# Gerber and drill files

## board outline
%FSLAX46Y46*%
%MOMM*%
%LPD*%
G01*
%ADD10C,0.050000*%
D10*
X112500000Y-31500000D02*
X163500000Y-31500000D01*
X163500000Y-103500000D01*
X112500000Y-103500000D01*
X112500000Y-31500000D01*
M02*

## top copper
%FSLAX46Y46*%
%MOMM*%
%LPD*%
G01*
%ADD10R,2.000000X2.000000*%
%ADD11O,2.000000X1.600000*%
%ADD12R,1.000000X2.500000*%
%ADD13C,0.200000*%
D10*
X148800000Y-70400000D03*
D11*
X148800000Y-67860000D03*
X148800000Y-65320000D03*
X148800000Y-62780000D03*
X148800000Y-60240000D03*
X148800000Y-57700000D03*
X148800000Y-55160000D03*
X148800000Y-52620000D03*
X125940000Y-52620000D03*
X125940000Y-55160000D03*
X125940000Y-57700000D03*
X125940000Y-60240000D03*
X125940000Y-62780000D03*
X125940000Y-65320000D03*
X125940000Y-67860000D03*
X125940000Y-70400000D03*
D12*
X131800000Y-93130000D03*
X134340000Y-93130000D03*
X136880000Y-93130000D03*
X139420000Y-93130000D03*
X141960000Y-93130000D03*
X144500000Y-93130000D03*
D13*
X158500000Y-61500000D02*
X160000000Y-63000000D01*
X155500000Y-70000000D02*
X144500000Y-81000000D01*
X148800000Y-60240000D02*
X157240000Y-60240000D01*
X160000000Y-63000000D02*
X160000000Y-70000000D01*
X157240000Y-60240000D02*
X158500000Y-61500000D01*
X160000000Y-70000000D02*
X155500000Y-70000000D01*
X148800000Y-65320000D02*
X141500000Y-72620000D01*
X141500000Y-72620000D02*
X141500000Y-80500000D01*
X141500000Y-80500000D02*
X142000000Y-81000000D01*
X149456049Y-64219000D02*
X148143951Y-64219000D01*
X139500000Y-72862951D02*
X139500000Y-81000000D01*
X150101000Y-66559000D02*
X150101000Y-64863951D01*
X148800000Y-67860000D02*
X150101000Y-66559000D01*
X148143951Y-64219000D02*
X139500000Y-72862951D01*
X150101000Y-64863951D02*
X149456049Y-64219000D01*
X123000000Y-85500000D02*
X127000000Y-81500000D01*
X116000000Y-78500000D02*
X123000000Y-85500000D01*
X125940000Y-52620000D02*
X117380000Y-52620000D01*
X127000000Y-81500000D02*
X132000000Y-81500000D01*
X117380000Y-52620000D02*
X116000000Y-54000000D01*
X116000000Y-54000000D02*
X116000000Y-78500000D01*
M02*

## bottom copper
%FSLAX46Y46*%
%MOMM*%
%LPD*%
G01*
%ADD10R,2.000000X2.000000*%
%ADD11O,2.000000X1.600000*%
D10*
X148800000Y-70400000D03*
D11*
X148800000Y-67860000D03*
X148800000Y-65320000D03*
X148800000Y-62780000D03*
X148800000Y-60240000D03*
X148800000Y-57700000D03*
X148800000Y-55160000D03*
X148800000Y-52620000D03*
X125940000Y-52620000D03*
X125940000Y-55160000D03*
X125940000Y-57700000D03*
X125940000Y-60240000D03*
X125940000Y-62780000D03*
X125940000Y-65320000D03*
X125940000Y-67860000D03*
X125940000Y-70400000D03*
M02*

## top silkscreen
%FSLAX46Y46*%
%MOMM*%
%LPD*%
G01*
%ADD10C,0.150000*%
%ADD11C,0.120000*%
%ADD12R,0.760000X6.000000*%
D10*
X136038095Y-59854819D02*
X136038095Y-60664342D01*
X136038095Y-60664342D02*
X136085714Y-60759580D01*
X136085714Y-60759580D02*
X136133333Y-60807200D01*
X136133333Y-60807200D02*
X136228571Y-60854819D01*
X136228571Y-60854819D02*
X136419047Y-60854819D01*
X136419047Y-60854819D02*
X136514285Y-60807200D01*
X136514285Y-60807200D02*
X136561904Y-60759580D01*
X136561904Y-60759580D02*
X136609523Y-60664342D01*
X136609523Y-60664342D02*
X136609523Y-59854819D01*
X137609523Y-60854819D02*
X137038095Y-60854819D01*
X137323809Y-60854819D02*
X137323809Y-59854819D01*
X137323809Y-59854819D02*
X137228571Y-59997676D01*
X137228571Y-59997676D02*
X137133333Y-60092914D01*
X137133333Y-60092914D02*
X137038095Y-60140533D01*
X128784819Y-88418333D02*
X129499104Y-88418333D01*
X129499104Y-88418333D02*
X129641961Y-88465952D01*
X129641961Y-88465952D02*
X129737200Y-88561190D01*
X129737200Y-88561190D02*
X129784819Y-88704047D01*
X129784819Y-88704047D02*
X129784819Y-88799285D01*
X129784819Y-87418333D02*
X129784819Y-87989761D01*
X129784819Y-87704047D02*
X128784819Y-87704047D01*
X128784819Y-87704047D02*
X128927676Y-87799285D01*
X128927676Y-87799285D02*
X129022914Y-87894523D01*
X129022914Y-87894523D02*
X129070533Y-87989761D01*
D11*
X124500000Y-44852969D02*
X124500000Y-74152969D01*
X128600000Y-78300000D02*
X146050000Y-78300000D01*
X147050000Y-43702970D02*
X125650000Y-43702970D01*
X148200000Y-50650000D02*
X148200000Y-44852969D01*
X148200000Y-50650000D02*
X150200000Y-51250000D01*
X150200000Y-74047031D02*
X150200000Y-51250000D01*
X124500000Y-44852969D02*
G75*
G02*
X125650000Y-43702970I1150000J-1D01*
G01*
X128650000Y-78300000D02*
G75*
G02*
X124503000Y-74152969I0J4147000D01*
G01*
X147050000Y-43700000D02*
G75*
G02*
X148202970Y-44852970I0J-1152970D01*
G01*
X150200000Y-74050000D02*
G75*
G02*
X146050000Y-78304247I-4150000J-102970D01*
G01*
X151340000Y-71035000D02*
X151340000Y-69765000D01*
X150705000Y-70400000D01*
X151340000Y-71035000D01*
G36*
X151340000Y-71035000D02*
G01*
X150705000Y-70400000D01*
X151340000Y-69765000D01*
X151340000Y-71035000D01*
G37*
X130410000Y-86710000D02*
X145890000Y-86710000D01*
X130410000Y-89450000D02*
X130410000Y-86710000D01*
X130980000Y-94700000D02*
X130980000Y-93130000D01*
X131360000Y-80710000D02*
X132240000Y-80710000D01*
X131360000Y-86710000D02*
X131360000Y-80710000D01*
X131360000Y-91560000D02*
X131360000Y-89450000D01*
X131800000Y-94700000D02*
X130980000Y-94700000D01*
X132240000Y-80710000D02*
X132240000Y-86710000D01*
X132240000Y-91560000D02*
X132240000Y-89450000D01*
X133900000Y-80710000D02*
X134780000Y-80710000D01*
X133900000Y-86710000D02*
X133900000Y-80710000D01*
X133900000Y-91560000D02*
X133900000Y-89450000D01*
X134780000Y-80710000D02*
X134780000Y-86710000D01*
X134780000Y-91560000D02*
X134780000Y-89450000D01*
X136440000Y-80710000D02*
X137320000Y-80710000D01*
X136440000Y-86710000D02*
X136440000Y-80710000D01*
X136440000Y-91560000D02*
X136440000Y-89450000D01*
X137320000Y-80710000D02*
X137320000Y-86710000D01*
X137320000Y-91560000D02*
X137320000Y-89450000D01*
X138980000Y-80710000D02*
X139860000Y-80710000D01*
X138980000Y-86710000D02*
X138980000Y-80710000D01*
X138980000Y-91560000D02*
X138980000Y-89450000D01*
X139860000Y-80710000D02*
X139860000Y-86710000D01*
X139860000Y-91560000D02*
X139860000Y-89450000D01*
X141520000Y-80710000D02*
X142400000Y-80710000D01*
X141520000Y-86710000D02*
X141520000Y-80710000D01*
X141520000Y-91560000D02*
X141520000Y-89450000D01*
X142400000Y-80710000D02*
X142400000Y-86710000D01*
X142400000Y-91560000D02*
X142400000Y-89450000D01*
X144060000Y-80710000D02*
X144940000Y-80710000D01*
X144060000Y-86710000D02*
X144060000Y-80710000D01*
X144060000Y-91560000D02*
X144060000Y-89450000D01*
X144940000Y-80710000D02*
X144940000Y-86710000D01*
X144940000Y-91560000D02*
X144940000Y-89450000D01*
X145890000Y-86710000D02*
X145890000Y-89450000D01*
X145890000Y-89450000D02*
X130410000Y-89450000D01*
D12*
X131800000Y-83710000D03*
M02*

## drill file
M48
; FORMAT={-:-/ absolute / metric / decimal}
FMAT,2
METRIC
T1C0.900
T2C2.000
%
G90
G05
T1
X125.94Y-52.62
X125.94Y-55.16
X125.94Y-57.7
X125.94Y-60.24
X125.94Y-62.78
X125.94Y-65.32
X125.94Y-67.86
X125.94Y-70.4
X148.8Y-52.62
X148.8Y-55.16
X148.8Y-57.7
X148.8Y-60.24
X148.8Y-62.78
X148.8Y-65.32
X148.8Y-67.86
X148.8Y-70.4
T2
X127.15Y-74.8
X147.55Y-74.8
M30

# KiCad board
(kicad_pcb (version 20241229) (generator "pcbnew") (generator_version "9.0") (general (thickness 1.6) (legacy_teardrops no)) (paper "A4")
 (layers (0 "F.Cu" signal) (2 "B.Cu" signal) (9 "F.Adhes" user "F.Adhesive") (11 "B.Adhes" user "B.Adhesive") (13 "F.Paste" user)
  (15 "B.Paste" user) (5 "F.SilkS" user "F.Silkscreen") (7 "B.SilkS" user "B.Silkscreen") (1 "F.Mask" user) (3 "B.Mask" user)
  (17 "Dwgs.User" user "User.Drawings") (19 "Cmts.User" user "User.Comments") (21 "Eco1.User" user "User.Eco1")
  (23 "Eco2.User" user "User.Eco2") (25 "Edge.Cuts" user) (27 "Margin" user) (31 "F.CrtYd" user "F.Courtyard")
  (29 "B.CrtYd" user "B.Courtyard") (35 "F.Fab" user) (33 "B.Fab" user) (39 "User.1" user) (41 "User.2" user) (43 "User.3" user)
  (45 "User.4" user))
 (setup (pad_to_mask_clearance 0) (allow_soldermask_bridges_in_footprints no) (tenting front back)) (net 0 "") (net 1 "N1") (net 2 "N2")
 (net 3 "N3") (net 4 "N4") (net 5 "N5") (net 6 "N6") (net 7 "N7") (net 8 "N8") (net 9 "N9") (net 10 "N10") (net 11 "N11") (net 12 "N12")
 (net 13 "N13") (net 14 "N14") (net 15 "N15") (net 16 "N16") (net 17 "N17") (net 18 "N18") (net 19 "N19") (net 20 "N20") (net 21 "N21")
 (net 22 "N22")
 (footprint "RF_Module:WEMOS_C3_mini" (layer "F.Cu") (at 148.8 70.4 180)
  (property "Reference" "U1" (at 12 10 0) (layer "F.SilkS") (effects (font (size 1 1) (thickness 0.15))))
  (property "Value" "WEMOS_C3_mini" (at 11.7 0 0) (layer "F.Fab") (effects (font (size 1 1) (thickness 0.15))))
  (fp_line (start 24.3 25.547031) (end 24.3 -3.752969) (stroke (width 0.12) (type solid)) (layer "F.SilkS"))
  (fp_line (start 20.2 -7.9) (end 2.75 -7.9) (stroke (width 0.12) (type solid)) (layer "F.SilkS"))
  (fp_line (start 1.75 26.69703) (end 23.15 26.69703) (stroke (width 0.12) (type solid)) (layer "F.SilkS"))
  (fp_line (start 0.6 19.75) (end 0.6 25.547031) (stroke (width 0.12) (type solid)) (layer "F.SilkS"))
  (fp_line (start 0.6 19.75) (end -1.4 19.15) (stroke (width 0.12) (type default)) (layer "F.SilkS"))
  (fp_line (start -1.4 -3.647031) (end -1.4 19.15) (stroke (width 0.12) (type solid)) (layer "F.SilkS"))
  (fp_arc (start 24.3 25.547031) (mid 23.963172 26.360203) (end 23.15 26.69703) (stroke (width 0.12) (type solid)) (layer "F.SilkS"))
  (fp_arc (start 20.15 -7.9) (mid 23.082383 -6.685361) (end 24.297 -3.752969) (stroke (width 0.12) (type solid)) (layer "F.SilkS"))
  (fp_arc (start 1.75 26.7) (mid 0.934727 26.362303) (end 0.59703 25.54703) (stroke (width 0.12) (type solid)) (layer "F.SilkS"))
  (fp_arc (start -1.4 -3.65) (mid -0.221578 -6.651732) (end 2.75 -7.904246) (stroke (width 0.12) (type solid)) (layer "F.SilkS"))
  (fp_poly (pts (xy -2.54 -0.635) (xy -2.54 0.635) (xy -1.905 0)) (stroke (width 0.12) (type solid)) (fill yes) (layer "F.SilkS"))
  (pad "" np_thru_hole circle (at 1.25 -4.4 180) (size 3 3) (drill 2) (layers "*.Mask"))
  (pad "" np_thru_hole circle (at 21.65 -4.4 180) (size 3 3) (drill 2) (layers "*.Mask"))
  (pad "1" thru_hole rect (at 0 0 180) (size 2 2) (drill 0.9) (layers "*.Cu" "*.Mask") (remove_unused_layers no) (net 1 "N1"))
  (pad "2" thru_hole oval (at 0 2.54 180) (size 2 1.6) (drill 0.9) (layers "*.Cu" "*.Mask") (remove_unused_layers no) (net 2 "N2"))
  (pad "3" thru_hole oval (at 0 5.08 180) (size 2 1.6) (drill 0.9) (layers "*.Cu" "*.Mask") (remove_unused_layers no) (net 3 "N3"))
  (pad "4" thru_hole oval (at 0 7.62 180) (size 2 1.6) (drill 0.9) (layers "*.Cu" "*.Mask") (remove_unused_layers no) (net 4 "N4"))
  (pad "5" thru_hole oval (at 0 10.16 180) (size 2 1.6) (drill 0.9) (layers "*.Cu" "*.Mask") (remove_unused_layers no) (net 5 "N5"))
  (pad "6" thru_hole oval (at 0 12.7 180) (size 2 1.6) (drill 0.9) (layers "*.Cu" "*.Mask") (remove_unused_layers no) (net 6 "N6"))
  (pad "7" thru_hole oval (at 0 15.24 180) (size 2 1.6) (drill 0.9) (layers "*.Cu" "*.Mask") (remove_unused_layers no) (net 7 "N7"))
  (pad "8" thru_hole oval (at 0 17.78 180) (size 2 1.6) (drill 0.9) (layers "*.Cu" "*.Mask") (remove_unused_layers no) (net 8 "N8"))
  (pad "9" thru_hole oval (at 22.86 17.78 180) (size 2 1.6) (drill 0.9) (layers "*.Cu" "*.Mask") (remove_unused_layers no) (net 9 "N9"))
  (pad "10" thru_hole oval (at 22.86 15.24 180) (size 2 1.6) (drill 0.9) (layers "*.Cu" "*.Mask") (remove_unused_layers no) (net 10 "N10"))
  (pad "11" thru_hole oval (at 22.86 12.7 180) (size 2 1.6) (drill 0.9) (layers "*.Cu" "*.Mask") (remove_unused_layers no) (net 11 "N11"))
  (pad "12" thru_hole oval (at 22.86 10.16 180) (size 2 1.6) (drill 0.9) (layers "*.Cu" "*.Mask") (remove_unused_layers no) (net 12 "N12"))
  (pad "13" thru_hole oval (at 22.86 7.62 180) (size 2 1.6) (drill 0.9) (layers "*.Cu" "*.Mask") (remove_unused_layers no) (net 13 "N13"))
  (pad "14" thru_hole oval (at 22.86 5.08 180) (size 2 1.6) (drill 0.9) (layers "*.Cu" "*.Mask") (remove_unused_layers no) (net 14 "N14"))
  (pad "15" thru_hole oval (at 22.86 2.54 180) (size 2 1.6) (drill 0.9) (layers "*.Cu" "*.Mask") (remove_unused_layers no) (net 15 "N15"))
  (pad "16" thru_hole oval (at 22.86 0 180) (size 2 1.6) (drill 0.9) (layers "*.Cu" "*.Mask") (remove_unused_layers no) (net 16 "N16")))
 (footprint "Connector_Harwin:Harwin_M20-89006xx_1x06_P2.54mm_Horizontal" (layer "F.Cu") (at 138.15 87.605 90)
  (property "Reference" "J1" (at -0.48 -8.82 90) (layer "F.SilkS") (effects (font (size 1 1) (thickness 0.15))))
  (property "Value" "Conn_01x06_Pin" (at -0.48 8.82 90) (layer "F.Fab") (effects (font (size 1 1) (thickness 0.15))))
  (fp_line (start 0.895 -7.74) (end 0.895 7.74) (stroke (width 0.12) (type solid)) (layer "F.SilkS"))
  (fp_line (start -1.845 -7.74) (end 0.895 -7.74) (stroke (width 0.12) (type solid)) (layer "F.SilkS"))
  (fp_line (start -7.095 -7.17) (end -5.525 -7.17) (stroke (width 0.12) (type solid)) (layer "F.SilkS"))
  (fp_line (start 6.895 -6.79) (end 6.895 -5.91) (stroke (width 0.12) (type solid)) (layer "F.SilkS"))
  (fp_line (start 0.895 -6.79) (end 6.895 -6.79) (stroke (width 0.12) (type solid)) (layer "F.SilkS"))
  (fp_line (start -3.955 -6.79) (end -1.845 -6.79) (stroke (width 0.12) (type solid)) (layer "F.SilkS"))
  (fp_line (start -7.095 -6.35) (end -7.095 -7.17) (stroke (width 0.12) (type solid)) (layer "F.SilkS"))
  (fp_line (start 6.895 -5.91) (end 0.895 -5.91) (stroke (width 0.12) (type solid)) (layer "F.SilkS"))
  (fp_line (start -3.955 -5.91) (end -1.845 -5.91) (stroke (width 0.12) (type solid)) (layer "F.SilkS"))
  (fp_line (start 6.895 -4.25) (end 6.895 -3.37) (stroke (width 0.12) (type solid)) (layer "F.SilkS"))
  (fp_line (start 0.895 -4.25) (end 6.895 -4.25) (stroke (width 0.12) (type solid)) (layer "F.SilkS"))
  (fp_line (start -3.955 -4.25) (end -1.845 -4.25) (stroke (width 0.12) (type solid)) (layer "F.SilkS"))
  (fp_line (start 6.895 -3.37) (end 0.895 -3.37) (stroke (width 0.12) (type solid)) (layer "F.SilkS"))
  (fp_line (start -3.955 -3.37) (end -1.845 -3.37) (stroke (width 0.12) (type solid)) (layer "F.SilkS"))
  (fp_line (start 6.895 -1.71) (end 6.895 -0.83) (stroke (width 0.12) (type solid)) (layer "F.SilkS"))
  (fp_line (start 0.895 -1.71) (end 6.895 -1.71) (stroke (width 0.12) (type solid)) (layer "F.SilkS"))
  (fp_line (start -3.955 -1.71) (end -1.845 -1.71) (stroke (width 0.12) (type solid)) (layer "F.SilkS"))
  (fp_line (start 6.895 -0.83) (end 0.895 -0.83) (stroke (width 0.12) (type solid)) (layer "F.SilkS"))
  (fp_line (start -3.955 -0.83) (end -1.845 -0.83) (stroke (width 0.12) (type solid)) (layer "F.SilkS"))
  (fp_line (start 6.895 0.83) (end 6.895 1.71) (stroke (width 0.12) (type solid)) (layer "F.SilkS"))
  (fp_line (start 0.895 0.83) (end 6.895 0.83) (stroke (width 0.12) (type solid)) (layer "F.SilkS"))
  (fp_line (start -3.955 0.83) (end -1.845 0.83) (stroke (width 0.12) (type solid)) (layer "F.SilkS"))
  (fp_line (start 6.895 1.71) (end 0.895 1.71) (stroke (width 0.12) (type solid)) (layer "F.SilkS"))
  (fp_line (start -3.955 1.71) (end -1.845 1.71) (stroke (width 0.12) (type solid)) (layer "F.SilkS"))
  (fp_line (start 6.895 3.37) (end 6.895 4.25) (stroke (width 0.12) (type solid)) (layer "F.SilkS"))
  (fp_line (start 0.895 3.37) (end 6.895 3.37) (stroke (width 0.12) (type solid)) (layer "F.SilkS"))
  (fp_line (start -3.955 3.37) (end -1.845 3.37) (stroke (width 0.12) (type solid)) (layer "F.SilkS"))
  (fp_line (start 6.895 4.25) (end 0.895 4.25) (stroke (width 0.12) (type solid)) (layer "F.SilkS"))
  (fp_line (start -3.955 4.25) (end -1.845 4.25) (stroke (width 0.12) (type solid)) (layer "F.SilkS"))
  (fp_line (start 6.895 5.91) (end 6.895 6.79) (stroke (width 0.12) (type solid)) (layer "F.SilkS"))
  (fp_line (start 0.895 5.91) (end 6.895 5.91) (stroke (width 0.12) (type solid)) (layer "F.SilkS"))
  (fp_line (start -3.955 5.91) (end -1.845 5.91) (stroke (width 0.12) (type solid)) (layer "F.SilkS"))
  (fp_line (start 6.895 6.79) (end 0.895 6.79) (stroke (width 0.12) (type solid)) (layer "F.SilkS"))
  (fp_line (start -3.955 6.79) (end -1.845 6.79) (stroke (width 0.12) (type solid)) (layer "F.SilkS"))
  (fp_line (start 0.895 7.74) (end -1.845 7.74) (stroke (width 0.12) (type solid)) (layer "F.SilkS"))
  (fp_line (start -1.845 7.74) (end -1.845 -7.74) (stroke (width 0.12) (type solid)) (layer "F.SilkS"))
  (pad "" smd rect (at 3.895 -6.35 90) (size 6 0.76) (layers "F.SilkS"))
  (pad "1" smd rect (at -5.525 -6.35 90) (size 2.5 1) (layers "F.Cu" "F.Mask" "F.Paste") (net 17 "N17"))
  (pad "2" smd rect (at -5.525 -3.81 90) (size 2.5 1) (layers "F.Cu" "F.Mask" "F.Paste") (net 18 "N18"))
  (pad "3" smd rect (at -5.525 -1.27 90) (size 2.5 1) (layers "F.Cu" "F.Mask" "F.Paste") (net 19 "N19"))
  (pad "4" smd rect (at -5.525 1.27 90) (size 2.5 1) (layers "F.Cu" "F.Mask" "F.Paste") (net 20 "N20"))
  (pad "5" smd rect (at -5.525 3.81 90) (size 2.5 1) (layers "F.Cu" "F.Mask" "F.Paste") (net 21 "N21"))
  (pad "6" smd rect (at -5.525 6.35 90) (size 2.5 1) (layers "F.Cu" "F.Mask" "F.Paste") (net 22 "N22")))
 (gr_rect (start 112.5 31.5) (end 163.5 103.5) (stroke (width 0.05) (type default)) (fill no) (layer "Edge.Cuts"))
 (segment (start 158.5 61.5) (end 160 63) (width 0.2) (layer "F.Cu") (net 5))
 (segment (start 155.5 70) (end 144.5 81) (width 0.2) (layer "F.Cu") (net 5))
 (segment (start 148.8 60.24) (end 157.24 60.24) (width 0.2) (layer "F.Cu") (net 5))
 (segment (start 160 63) (end 160 70) (width 0.2) (layer "F.Cu") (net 5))
 (segment (start 157.24 60.24) (end 158.5 61.5) (width 0.2) (layer "F.Cu") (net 5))
 (segment (start 160 70) (end 155.5 70) (width 0.2) (layer "F.Cu") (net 5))
 (segment (start 148.8 65.32) (end 141.5 72.62) (width 0.2) (layer "F.Cu") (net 3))
 (segment (start 141.5 72.62) (end 141.5 80.5) (width 0.2) (layer "F.Cu") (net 3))
 (segment (start 141.5 80.5) (end 142 81) (width 0.2) (layer "F.Cu") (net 3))
 (segment (start 149.456049 64.219) (end 148.143951 64.219) (width 0.2) (layer "F.Cu") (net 2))
 (segment (start 139.5 72.862951) (end 139.5 81) (width 0.2) (layer "F.Cu") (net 2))
 (segment (start 150.101 66.559) (end 150.101 64.863951) (width 0.2) (layer "F.Cu") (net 2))
 (segment (start 148.8 67.86) (end 150.101 66.559) (width 0.2) (layer "F.Cu") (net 2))
 (segment (start 148.143951 64.219) (end 139.5 72.862951) (width 0.2) (layer "F.Cu") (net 2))
 (segment (start 150.101 64.863951) (end 149.456049 64.219) (width 0.2) (layer "F.Cu") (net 2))
 (segment (start 123 85.5) (end 127 81.5) (width 0.2) (layer "F.Cu") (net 9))
 (segment (start 116 78.5) (end 123 85.5) (width 0.2) (layer "F.Cu") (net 9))
 (segment (start 125.94 52.62) (end 117.38 52.62) (width 0.2) (layer "F.Cu") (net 9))
 (segment (start 127 81.5) (end 132 81.5) (width 0.2) (layer "F.Cu") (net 9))
 (segment (start 117.38 52.62) (end 116 54) (width 0.2) (layer "F.Cu") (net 9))
 (segment (start 116 54) (end 116 78.5) (width 0.2) (layer "F.Cu") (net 9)))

